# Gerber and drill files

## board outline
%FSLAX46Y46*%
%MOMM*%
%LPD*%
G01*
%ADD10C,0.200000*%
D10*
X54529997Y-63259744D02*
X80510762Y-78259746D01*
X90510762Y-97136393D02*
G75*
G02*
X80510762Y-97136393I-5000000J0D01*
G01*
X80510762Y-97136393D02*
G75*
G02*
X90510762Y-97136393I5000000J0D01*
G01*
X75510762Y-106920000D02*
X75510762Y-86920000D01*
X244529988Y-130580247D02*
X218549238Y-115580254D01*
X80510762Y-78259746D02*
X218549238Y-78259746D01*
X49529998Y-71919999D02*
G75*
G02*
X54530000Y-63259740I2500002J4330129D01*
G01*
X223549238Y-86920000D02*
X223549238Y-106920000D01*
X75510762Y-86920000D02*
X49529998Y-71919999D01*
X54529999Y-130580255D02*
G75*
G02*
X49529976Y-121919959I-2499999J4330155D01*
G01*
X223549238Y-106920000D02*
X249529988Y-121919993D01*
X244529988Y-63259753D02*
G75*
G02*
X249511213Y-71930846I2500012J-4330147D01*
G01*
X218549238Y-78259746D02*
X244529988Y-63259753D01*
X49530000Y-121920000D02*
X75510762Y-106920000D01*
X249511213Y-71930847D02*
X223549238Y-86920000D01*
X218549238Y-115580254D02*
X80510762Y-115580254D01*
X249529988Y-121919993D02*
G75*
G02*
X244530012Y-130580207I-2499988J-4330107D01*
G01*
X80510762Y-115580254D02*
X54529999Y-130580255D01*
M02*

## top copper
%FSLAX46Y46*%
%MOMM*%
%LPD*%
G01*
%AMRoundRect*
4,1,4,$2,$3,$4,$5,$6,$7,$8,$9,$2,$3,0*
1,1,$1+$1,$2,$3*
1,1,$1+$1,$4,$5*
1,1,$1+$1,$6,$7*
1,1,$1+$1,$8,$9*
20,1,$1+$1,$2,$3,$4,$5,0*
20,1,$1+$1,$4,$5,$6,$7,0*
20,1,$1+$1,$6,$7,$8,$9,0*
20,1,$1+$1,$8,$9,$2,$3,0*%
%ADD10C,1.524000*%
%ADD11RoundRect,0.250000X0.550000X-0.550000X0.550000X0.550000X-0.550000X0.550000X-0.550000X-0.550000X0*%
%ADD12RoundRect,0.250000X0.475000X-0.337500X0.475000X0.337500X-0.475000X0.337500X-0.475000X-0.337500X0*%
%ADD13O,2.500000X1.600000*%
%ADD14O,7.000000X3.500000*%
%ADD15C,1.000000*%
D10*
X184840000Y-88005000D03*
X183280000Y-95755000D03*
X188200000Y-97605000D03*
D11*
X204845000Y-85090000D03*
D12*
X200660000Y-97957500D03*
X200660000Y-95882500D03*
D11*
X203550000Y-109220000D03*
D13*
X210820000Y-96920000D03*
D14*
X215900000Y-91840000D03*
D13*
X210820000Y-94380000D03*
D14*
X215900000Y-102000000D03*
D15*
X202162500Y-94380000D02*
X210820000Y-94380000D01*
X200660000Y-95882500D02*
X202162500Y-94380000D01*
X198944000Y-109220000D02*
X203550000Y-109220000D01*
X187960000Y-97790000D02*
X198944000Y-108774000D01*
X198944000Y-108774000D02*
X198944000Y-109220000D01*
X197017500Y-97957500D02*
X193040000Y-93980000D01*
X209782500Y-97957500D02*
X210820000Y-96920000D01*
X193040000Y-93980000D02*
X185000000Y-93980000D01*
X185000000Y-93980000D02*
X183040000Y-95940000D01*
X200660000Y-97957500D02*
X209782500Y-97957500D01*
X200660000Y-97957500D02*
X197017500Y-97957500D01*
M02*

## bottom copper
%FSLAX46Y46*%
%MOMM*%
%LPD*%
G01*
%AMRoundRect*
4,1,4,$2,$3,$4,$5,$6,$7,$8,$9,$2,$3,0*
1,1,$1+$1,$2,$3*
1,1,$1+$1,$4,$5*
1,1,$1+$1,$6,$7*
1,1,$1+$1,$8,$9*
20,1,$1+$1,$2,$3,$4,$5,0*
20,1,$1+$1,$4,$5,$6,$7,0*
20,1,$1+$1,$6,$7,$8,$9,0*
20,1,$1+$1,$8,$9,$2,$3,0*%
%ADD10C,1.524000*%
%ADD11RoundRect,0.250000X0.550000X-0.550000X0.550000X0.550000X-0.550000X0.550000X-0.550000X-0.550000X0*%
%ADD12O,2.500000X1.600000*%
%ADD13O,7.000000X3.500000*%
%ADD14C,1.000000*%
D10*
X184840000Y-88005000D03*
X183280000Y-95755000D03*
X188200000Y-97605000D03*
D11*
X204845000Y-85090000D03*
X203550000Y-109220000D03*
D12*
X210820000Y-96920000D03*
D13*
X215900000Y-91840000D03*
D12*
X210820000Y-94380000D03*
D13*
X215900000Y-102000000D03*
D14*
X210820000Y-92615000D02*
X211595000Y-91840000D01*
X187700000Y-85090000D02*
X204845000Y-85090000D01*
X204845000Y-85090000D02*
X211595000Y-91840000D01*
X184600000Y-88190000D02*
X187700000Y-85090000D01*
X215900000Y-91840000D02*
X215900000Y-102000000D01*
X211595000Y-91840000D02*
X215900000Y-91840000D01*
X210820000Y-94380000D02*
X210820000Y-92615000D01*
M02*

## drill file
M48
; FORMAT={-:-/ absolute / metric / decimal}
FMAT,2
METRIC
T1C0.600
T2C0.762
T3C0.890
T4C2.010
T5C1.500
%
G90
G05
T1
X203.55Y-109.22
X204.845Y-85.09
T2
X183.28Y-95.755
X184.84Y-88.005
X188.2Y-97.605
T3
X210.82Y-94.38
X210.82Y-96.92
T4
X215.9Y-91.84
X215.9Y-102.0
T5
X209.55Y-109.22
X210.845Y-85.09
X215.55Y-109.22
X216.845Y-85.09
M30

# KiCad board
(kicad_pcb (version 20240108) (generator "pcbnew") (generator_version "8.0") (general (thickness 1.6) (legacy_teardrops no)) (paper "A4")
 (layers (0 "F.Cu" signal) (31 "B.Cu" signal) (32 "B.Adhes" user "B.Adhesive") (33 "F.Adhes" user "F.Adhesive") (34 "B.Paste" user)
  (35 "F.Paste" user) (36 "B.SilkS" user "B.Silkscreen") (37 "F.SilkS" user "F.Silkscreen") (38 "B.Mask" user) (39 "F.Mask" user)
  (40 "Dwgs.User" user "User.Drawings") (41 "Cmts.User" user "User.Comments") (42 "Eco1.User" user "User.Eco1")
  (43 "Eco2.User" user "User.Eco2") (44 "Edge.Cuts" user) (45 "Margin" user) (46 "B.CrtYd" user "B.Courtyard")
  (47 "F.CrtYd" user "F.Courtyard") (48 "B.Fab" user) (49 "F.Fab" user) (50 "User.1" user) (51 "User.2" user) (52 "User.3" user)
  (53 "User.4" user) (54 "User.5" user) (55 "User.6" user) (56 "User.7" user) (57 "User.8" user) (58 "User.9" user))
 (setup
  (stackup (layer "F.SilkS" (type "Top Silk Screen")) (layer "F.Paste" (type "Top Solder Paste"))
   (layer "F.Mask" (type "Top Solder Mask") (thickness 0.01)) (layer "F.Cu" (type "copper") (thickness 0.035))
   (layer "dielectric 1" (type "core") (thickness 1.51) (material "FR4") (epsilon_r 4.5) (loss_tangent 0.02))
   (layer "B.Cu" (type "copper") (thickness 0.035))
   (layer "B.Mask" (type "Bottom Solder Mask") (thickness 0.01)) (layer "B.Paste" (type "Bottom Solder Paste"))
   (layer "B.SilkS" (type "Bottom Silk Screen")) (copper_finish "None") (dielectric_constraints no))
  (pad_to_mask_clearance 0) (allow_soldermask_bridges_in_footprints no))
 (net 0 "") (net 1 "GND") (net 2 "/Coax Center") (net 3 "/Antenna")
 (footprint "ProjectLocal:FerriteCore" (layer "F.Cu") (at 173.99 97.155 -90)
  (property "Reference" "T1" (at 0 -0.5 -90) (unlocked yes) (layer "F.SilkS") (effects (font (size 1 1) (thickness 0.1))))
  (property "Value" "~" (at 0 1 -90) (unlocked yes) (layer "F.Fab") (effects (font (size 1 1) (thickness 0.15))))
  (pad "1" thru_hole circle (at -9.15 -10.85 270) (size 1.524 1.524) (drill 0.762) (layers "*.Cu" "*.Mask") (remove_unused_layers no)
   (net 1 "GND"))
  (pad "2" thru_hole circle (at -1.4 -9.29 270) (size 1.524 1.524) (drill 0.762) (layers "*.Cu" "*.Mask") (remove_unused_layers no)
   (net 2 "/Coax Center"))
  (pad "3" thru_hole circle (at 0.45 -14.21 270) (size 1.524 1.524) (drill 0.762) (layers "*.Cu" "*.Mask") (remove_unused_layers no)
   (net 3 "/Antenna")))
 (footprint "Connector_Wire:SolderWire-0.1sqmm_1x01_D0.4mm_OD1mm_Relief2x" (layer "F.Cu") (at 204.845 85.09 90)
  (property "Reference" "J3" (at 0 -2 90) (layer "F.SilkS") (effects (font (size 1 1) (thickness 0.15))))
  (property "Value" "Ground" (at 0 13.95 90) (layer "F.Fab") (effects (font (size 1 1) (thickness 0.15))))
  (pad "" np_thru_hole circle (at 0 6 90) (size 1.5 1.5) (drill 1.5) (layers "*.Cu" "*.Mask"))
  (pad "" np_thru_hole circle (at 0 12 90) (size 1.5 1.5) (drill 1.5) (layers "*.Cu" "*.Mask"))
  (pad "1" thru_hole roundrect (at 0 0 90) (size 1.6 1.6) (drill 0.6) (layers "*.Cu" "*.Mask") (remove_unused_layers no)
   (roundrect_rratio 0.15625) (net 1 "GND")))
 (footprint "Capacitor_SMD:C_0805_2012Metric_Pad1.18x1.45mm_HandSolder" (layer "F.Cu") (at 200.66 96.92 90)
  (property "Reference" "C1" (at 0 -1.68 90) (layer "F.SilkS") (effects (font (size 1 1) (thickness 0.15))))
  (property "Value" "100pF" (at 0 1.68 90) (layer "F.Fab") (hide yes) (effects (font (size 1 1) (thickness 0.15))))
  (pad "1" smd roundrect (at -1.0375 0 90) (size 1.175 1.45) (layers "F.Cu" "F.Paste" "F.Mask") (roundrect_rratio 0.212766)
   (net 2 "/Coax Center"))
  (pad "2" smd roundrect (at 1.0375 0 90) (size 1.175 1.45) (layers "F.Cu" "F.Paste" "F.Mask") (roundrect_rratio 0.212766) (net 1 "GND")))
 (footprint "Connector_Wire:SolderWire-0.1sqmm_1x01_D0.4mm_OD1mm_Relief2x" (layer "F.Cu") (at 203.55 109.22 90)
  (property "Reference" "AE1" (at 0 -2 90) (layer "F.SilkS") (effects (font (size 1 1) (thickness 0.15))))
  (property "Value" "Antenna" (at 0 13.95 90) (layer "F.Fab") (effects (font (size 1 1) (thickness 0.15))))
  (pad "" np_thru_hole circle (at 0 6 90) (size 1.5 1.5) (drill 1.5) (layers "*.Cu" "*.Mask"))
  (pad "" np_thru_hole circle (at 0 12 90) (size 1.5 1.5) (drill 1.5) (layers "*.Cu" "*.Mask"))
  (pad "1" thru_hole roundrect (at 0 0 90) (size 1.6 1.6) (drill 0.6) (layers "*.Cu" "*.Mask") (remove_unused_layers no)
   (roundrect_rratio 0.15625) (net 3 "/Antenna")))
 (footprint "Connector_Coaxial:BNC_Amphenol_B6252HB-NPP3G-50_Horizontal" (layer "F.Cu") (at 210.82 96.92 -90)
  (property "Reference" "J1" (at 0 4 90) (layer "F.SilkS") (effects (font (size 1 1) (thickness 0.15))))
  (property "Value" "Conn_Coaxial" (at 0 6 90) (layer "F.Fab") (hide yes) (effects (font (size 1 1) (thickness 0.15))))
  (pad "1" thru_hole oval (at 0 0 270) (size 1.6 2.5) (drill 0.89) (layers "*.Cu" "*.Mask") (remove_unused_layers no) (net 2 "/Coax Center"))
  (pad "2" thru_hole oval (at -5.08 -5.08 270) (size 3.5 7) (drill 2.01) (layers "*.Cu" "*.Mask") (remove_unused_layers no) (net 1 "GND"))
  (pad "2" thru_hole oval (at -2.54 0 270) (size 1.6 2.5) (drill 0.89) (layers "*.Cu" "*.Mask") (remove_unused_layers no) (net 1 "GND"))
  (pad "2" thru_hole oval (at 5.08 -5.08 270) (size 3.5 7) (drill 2.01) (layers "*.Cu" "*.Mask") (remove_unused_layers no) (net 1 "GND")))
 (gr_line (start 54.529997 63.259744) (end 80.510762 78.259746) (stroke (width 0.2) (type default)) (layer "Edge.Cuts"))
 (gr_circle (center 85.510762 97.136393) (end 90.510762 97.136393) (stroke (width 0.2) (type default)) (fill none) (layer "Edge.Cuts"))
 (gr_line (start 75.510762 106.92) (end 75.510762 86.92) (stroke (width 0.2) (type default)) (layer "Edge.Cuts"))
 (gr_line (start 244.529988 130.580247) (end 218.549238 115.580254) (stroke (width 0.2) (type default)) (layer "Edge.Cuts"))
 (gr_line (start 80.510762 78.259746) (end 218.549238 78.259746) (stroke (width 0.2) (type default)) (layer "Edge.Cuts"))
 (gr_arc (start 49.529998 71.919999) (mid 47.699869 65.089871) (end 54.529997 63.259744) (stroke (width 0.2) (type default))
  (layer "Edge.Cuts"))
 (gr_line (start 223.549238 86.92) (end 223.549238 106.92) (stroke (width 0.2) (type default)) (layer "Edge.Cuts"))
 (gr_line (start 75.510762 86.92) (end 49.529998 71.919999) (stroke (width 0.2) (type default)) (layer "Edge.Cuts"))
 (gr_arc (start 54.529999 130.580255) (mid 47.699875 128.750128) (end 49.53 121.92) (stroke (width 0.2) (type default)) (layer "Edge.Cuts"))
 (gr_line (start 223.549238 106.92) (end 249.529988 121.919993) (stroke (width 0.2) (type default)) (layer "Edge.Cuts"))
 (gr_arc (start 244.529988 63.259753) (mid 251.365557 65.099282) (end 249.511213 71.930847) (stroke (width 0.2) (type default))
  (layer "Edge.Cuts"))
 (gr_line (start 218.549238 78.259746) (end 244.529988 63.259753) (stroke (width 0.2) (type default)) (layer "Edge.Cuts"))
 (gr_line (start 49.53 121.92) (end 75.510762 106.92) (stroke (width 0.2) (type default)) (layer "Edge.Cuts"))
 (gr_line (start 249.511213 71.930847) (end 223.549238 86.92) (stroke (width 0.2) (type default)) (layer "Edge.Cuts"))
 (gr_line (start 218.549238 115.580254) (end 80.510762 115.580254) (stroke (width 0.2) (type default)) (layer "Edge.Cuts"))
 (gr_arc (start 249.529988 121.919993) (mid 251.360107 128.750088) (end 244.530012 130.580206) (stroke (width 0.2) (type default))
  (layer "Edge.Cuts"))
 (gr_line (start 80.510762 115.580254) (end 54.529999 130.580255) (stroke (width 0.2) (type default)) (layer "Edge.Cuts"))
 (segment (start 202.1625 94.38) (end 210.82 94.38) (width 1) (layer "F.Cu") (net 1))
 (segment (start 200.66 95.8825) (end 202.1625 94.38) (width 1) (layer "F.Cu") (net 1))
 (segment (start 210.82 92.615) (end 211.595 91.84) (width 1) (layer "B.Cu") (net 1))
 (segment (start 187.7 85.09) (end 204.845 85.09) (width 1) (layer "B.Cu") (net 1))
 (segment (start 204.845 85.09) (end 211.595 91.84) (width 1) (layer "B.Cu") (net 1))
 (segment (start 184.6 88.19) (end 187.7 85.09) (width 1) (layer "B.Cu") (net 1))
 (segment (start 215.9 91.84) (end 215.9 102) (width 1) (layer "B.Cu") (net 1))
 (segment (start 211.595 91.84) (end 215.9 91.84) (width 1) (layer "B.Cu") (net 1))
 (segment (start 210.82 94.38) (end 210.82 92.615) (width 1) (layer "B.Cu") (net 1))
 (segment (start 198.944 109.22) (end 203.55 109.22) (width 1) (layer "F.Cu") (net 3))
 (segment (start 187.96 97.79) (end 198.944 108.774) (width 1) (layer "F.Cu") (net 3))
 (segment (start 198.944 108.774) (end 198.944 109.22) (width 1) (layer "F.Cu") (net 3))
 (segment (start 197.0175 97.9575) (end 193.04 93.98) (width 1) (layer "F.Cu") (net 2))
 (segment (start 209.7825 97.9575) (end 210.82 96.92) (width 1) (layer "F.Cu") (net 2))
 (segment (start 193.04 93.98) (end 185 93.98) (width 1) (layer "F.Cu") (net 2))
 (segment (start 185 93.98) (end 183.04 95.94) (width 1) (layer "F.Cu") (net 2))
 (segment (start 200.66 97.9575) (end 209.7825 97.9575) (width 1) (layer "F.Cu") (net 2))
 (segment (start 200.66 97.9575) (end 197.0175 97.9575) (width 1) (layer "F.Cu") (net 2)))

